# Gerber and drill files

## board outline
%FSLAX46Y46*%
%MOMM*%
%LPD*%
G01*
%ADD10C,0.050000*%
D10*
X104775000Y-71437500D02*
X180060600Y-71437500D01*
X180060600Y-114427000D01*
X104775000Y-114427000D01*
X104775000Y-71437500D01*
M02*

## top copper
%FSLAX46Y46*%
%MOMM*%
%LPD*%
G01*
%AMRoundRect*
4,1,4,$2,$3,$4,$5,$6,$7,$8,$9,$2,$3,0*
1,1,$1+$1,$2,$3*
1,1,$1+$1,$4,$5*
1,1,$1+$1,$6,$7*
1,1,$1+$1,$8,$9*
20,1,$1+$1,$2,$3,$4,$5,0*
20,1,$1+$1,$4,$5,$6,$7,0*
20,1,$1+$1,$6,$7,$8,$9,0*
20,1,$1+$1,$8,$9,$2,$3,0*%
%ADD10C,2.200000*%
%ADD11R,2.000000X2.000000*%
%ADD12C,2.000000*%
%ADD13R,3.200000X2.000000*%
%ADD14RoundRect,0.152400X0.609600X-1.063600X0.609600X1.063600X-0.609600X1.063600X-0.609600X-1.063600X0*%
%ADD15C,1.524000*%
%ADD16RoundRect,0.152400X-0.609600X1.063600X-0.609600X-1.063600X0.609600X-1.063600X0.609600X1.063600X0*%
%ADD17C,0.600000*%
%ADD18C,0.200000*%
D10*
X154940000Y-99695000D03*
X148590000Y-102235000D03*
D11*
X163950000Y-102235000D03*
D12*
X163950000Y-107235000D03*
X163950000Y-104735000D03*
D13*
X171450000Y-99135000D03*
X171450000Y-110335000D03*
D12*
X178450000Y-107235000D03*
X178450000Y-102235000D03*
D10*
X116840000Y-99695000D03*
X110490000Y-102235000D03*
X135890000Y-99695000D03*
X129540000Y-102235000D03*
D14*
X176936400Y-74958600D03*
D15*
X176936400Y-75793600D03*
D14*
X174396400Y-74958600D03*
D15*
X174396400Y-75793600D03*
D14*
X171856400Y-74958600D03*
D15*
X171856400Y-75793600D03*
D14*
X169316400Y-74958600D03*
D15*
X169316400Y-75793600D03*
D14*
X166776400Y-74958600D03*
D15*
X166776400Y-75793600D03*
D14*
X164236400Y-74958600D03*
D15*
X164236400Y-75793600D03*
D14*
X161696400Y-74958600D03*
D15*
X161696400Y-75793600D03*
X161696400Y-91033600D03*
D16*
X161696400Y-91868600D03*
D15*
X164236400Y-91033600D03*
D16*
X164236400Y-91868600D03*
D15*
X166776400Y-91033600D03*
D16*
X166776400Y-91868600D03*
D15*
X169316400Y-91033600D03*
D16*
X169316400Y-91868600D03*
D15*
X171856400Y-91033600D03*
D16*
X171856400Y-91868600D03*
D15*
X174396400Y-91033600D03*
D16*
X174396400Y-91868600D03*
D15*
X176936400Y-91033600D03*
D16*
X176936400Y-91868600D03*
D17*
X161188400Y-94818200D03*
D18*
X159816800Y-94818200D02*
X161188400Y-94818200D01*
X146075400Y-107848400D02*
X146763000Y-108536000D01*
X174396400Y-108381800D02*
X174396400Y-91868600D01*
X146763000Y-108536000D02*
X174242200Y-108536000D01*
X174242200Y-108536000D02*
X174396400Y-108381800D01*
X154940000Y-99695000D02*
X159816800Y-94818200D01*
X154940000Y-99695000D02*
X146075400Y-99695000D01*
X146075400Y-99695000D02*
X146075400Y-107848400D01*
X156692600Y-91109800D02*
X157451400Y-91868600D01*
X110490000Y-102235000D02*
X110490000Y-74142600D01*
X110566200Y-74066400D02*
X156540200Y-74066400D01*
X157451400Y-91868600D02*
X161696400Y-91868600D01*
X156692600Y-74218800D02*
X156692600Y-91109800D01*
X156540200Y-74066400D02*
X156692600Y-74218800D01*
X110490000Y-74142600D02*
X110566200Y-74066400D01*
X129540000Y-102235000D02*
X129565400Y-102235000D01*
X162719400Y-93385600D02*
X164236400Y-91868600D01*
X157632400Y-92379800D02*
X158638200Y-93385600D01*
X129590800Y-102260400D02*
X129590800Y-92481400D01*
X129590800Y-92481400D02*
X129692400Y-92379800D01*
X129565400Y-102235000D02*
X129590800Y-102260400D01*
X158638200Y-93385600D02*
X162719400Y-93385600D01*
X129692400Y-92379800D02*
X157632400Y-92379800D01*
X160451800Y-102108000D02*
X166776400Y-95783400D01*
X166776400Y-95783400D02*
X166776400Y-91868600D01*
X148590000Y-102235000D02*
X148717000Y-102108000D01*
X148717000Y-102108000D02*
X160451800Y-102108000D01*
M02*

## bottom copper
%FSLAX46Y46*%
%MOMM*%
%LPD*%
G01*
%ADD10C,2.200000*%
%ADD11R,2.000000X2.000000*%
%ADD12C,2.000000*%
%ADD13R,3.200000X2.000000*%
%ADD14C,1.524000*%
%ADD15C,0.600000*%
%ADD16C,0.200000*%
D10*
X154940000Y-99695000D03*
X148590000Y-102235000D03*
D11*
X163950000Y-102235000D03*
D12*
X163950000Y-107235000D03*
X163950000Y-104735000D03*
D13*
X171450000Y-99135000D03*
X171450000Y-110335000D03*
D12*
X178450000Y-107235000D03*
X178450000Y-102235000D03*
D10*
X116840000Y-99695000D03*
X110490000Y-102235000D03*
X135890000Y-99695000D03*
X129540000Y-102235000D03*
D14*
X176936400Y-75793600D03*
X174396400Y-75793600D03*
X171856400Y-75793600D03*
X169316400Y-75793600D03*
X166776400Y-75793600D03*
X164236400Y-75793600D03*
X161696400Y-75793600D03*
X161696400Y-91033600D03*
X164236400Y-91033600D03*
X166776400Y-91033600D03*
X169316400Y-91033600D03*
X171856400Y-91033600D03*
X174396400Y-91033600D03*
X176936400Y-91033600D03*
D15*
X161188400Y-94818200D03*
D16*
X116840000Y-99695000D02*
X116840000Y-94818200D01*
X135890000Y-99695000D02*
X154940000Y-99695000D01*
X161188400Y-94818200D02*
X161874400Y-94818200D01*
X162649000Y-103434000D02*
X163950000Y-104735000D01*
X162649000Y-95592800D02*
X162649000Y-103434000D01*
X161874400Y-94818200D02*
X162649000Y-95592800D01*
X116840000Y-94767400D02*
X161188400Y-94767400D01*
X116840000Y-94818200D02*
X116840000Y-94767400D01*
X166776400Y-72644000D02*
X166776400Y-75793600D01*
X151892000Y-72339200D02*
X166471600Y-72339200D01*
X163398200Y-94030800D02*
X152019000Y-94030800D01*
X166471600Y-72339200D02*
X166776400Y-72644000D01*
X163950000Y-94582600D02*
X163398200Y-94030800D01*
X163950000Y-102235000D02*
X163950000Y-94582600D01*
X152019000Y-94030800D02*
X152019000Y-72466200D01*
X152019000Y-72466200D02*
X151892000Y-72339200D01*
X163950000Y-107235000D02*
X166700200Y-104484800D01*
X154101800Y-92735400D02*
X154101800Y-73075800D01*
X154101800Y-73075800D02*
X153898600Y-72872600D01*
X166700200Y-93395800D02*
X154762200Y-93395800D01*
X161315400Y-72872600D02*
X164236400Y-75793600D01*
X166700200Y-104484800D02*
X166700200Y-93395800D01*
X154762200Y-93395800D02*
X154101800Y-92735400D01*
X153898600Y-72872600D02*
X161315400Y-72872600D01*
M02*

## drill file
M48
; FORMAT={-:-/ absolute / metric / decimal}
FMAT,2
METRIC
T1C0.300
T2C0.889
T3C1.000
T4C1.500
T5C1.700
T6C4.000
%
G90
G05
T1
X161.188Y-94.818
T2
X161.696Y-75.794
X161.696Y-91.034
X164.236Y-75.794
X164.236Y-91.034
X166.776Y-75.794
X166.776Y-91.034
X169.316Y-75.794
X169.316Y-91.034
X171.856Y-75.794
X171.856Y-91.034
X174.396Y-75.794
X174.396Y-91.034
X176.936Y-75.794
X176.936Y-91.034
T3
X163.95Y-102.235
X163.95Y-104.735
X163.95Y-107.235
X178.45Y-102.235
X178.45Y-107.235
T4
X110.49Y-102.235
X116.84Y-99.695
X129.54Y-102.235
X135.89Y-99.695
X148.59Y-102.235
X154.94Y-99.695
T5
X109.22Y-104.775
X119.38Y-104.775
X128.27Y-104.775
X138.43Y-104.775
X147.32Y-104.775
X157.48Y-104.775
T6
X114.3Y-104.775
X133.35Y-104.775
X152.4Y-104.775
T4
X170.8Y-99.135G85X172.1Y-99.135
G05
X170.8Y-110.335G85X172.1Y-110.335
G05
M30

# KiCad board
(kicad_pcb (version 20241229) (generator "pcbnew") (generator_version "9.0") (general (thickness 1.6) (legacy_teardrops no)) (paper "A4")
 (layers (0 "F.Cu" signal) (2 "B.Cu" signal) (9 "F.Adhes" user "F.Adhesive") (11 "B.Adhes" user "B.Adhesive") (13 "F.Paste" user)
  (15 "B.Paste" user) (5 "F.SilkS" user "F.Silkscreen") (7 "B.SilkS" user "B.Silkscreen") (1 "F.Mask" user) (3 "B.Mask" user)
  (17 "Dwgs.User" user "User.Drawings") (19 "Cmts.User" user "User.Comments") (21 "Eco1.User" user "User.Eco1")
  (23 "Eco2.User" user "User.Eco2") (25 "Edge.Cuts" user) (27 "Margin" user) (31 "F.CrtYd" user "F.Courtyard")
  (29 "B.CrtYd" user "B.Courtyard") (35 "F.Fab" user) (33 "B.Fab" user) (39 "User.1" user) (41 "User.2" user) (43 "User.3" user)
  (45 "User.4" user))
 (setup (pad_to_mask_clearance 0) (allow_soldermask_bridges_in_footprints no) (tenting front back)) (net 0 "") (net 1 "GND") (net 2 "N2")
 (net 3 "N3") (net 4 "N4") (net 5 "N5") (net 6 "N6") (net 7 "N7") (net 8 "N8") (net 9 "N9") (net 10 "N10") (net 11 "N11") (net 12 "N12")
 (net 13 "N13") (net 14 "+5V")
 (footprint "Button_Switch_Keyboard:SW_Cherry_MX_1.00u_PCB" (layer "F.Cu") (at 154.94 99.695)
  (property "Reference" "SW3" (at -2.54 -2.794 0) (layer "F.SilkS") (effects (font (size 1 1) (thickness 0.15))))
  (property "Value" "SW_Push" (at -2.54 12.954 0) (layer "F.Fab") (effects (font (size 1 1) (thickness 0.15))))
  (pad "" np_thru_hole circle (at -7.62 5.08) (size 1.7 1.7) (drill 1.7) (layers "*.Cu" "*.Mask"))
  (pad "" np_thru_hole circle (at -2.54 5.08) (size 4 4) (drill 4) (layers "*.Cu" "*.Mask"))
  (pad "" np_thru_hole circle (at 2.54 5.08) (size 1.7 1.7) (drill 1.7) (layers "*.Cu" "*.Mask"))
  (pad "1" thru_hole circle (at 0 0) (size 2.2 2.2) (drill 1.5) (layers "*.Cu" "*.Mask") (remove_unused_layers no) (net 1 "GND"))
  (pad "2" thru_hole circle (at -6.35 2.54) (size 2.2 2.2) (drill 1.5) (layers "*.Cu" "*.Mask") (remove_unused_layers no) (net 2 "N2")))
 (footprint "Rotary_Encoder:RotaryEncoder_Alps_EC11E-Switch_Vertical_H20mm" (layer "F.Cu") (at 163.95 102.235)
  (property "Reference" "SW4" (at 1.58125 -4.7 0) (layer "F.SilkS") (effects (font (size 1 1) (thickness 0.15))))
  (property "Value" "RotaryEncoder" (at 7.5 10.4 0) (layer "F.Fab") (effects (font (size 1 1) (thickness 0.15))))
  (pad "A" thru_hole rect (at 0 0) (size 2 2) (drill 1) (layers "*.Cu" "*.Mask") (remove_unused_layers no) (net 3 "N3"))
  (pad "B" thru_hole circle (at 0 5) (size 2 2) (drill 1) (layers "*.Cu" "*.Mask") (remove_unused_layers no) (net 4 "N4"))
  (pad "C" thru_hole circle (at 0 2.5) (size 2 2) (drill 1) (layers "*.Cu" "*.Mask") (remove_unused_layers no) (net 1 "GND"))
  (pad "MP" thru_hole rect (at 7.5 -3.1) (size 3.2 2) (drill oval 2.8 1.5) (layers "*.Cu" "*.Mask") (remove_unused_layers no))
  (pad "MP" thru_hole rect (at 7.5 8.1) (size 3.2 2) (drill oval 2.8 1.5) (layers "*.Cu" "*.Mask") (remove_unused_layers no))
  (pad "S1" thru_hole circle (at 14.5 5) (size 2 2) (drill 1) (layers "*.Cu" "*.Mask") (remove_unused_layers no))
  (pad "S2" thru_hole circle (at 14.5 0) (size 2 2) (drill 1) (layers "*.Cu" "*.Mask") (remove_unused_layers no)))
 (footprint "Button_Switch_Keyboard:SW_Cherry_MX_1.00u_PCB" (layer "F.Cu") (at 116.84 99.695)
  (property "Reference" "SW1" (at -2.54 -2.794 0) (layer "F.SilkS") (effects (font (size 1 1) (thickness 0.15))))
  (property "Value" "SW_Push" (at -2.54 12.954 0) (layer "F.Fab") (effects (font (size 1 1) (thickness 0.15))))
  (pad "" np_thru_hole circle (at -7.62 5.08) (size 1.7 1.7) (drill 1.7) (layers "*.Cu" "*.Mask"))
  (pad "" np_thru_hole circle (at -2.54 5.08) (size 4 4) (drill 4) (layers "*.Cu" "*.Mask"))
  (pad "" np_thru_hole circle (at 2.54 5.08) (size 1.7 1.7) (drill 1.7) (layers "*.Cu" "*.Mask"))
  (pad "1" thru_hole circle (at 0 0) (size 2.2 2.2) (drill 1.5) (layers "*.Cu" "*.Mask") (remove_unused_layers no) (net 1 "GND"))
  (pad "2" thru_hole circle (at -6.35 2.54) (size 2.2 2.2) (drill 1.5) (layers "*.Cu" "*.Mask") (remove_unused_layers no) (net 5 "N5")))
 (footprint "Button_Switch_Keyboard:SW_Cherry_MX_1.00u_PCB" (layer "F.Cu") (at 135.89 99.695)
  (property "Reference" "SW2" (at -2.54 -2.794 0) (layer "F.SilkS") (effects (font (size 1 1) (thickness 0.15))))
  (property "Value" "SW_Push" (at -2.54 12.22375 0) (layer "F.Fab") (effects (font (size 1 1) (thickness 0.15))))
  (pad "" np_thru_hole circle (at -7.62 5.08) (size 1.7 1.7) (drill 1.7) (layers "*.Cu" "*.Mask"))
  (pad "" np_thru_hole circle (at -2.54 5.08) (size 4 4) (drill 4) (layers "*.Cu" "*.Mask"))
  (pad "" np_thru_hole circle (at 2.54 5.08) (size 1.7 1.7) (drill 1.7) (layers "*.Cu" "*.Mask"))
  (pad "1" thru_hole circle (at 0 0) (size 2.2 2.2) (drill 1.5) (layers "*.Cu" "*.Mask") (remove_unused_layers no) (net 1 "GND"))
  (pad "2" thru_hole circle (at -6.35 2.54) (size 2.2 2.2) (drill 1.5) (layers "*.Cu" "*.Mask") (remove_unused_layers no) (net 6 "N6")))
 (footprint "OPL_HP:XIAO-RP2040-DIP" (layer "F.Cu") (at 169.3164 83.4136 -90)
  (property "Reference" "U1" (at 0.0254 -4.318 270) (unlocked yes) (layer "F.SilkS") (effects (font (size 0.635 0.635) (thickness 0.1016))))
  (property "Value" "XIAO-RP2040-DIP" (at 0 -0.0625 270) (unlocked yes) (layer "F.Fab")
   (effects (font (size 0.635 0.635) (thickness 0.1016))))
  (pad "1" smd roundrect (at -8.455 -7.62 90) (size 2.432 1.524) (layers "F.Cu" "F.Mask") (roundrect_rratio 0.1) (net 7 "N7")
   (thermal_bridge_angle 45))
  (pad "1" thru_hole circle (at -7.62 -7.62 90) (size 1.524 1.524) (drill 0.889) (layers "*.Cu" "*.Mask") (remove_unused_layers no)
   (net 7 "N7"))
  (pad "2" smd roundrect (at -8.455 -5.08 90) (size 2.432 1.524) (layers "F.Cu" "F.Mask") (roundrect_rratio 0.1) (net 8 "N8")
   (thermal_bridge_angle 45))
  (pad "2" thru_hole circle (at -7.62 -5.08 90) (size 1.524 1.524) (drill 0.889) (layers "*.Cu" "*.Mask") (remove_unused_layers no)
   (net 8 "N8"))
  (pad "3" smd roundrect (at -8.455 -2.54 90) (size 2.432 1.524) (layers "F.Cu" "F.Mask") (roundrect_rratio 0.1) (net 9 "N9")
   (thermal_bridge_angle 45))
  (pad "3" thru_hole circle (at -7.62 -2.54 90) (size 1.524 1.524) (drill 0.889) (layers "*.Cu" "*.Mask") (remove_unused_layers no)
   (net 9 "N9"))
  (pad "4" smd roundrect (at -8.455 0 90) (size 2.432 1.524) (layers "F.Cu" "F.Mask") (roundrect_rratio 0.1) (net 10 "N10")
   (thermal_bridge_angle 45))
  (pad "4" thru_hole circle (at -7.62 0 90) (size 1.524 1.524) (drill 0.889) (layers "*.Cu" "*.Mask") (remove_unused_layers no)
   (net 10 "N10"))
  (pad "5" smd roundrect (at -8.455 2.54 90) (size 2.432 1.524) (layers "F.Cu" "F.Mask") (roundrect_rratio 0.1) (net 3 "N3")
   (thermal_bridge_angle 45))
  (pad "5" thru_hole circle (at -7.62 2.54 90) (size 1.524 1.524) (drill 0.889) (layers "*.Cu" "*.Mask") (remove_unused_layers no)
   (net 3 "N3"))
  (pad "6" smd roundrect (at -8.455 5.08 90) (size 2.432 1.524) (layers "F.Cu" "F.Mask") (roundrect_rratio 0.1) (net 4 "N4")
   (thermal_bridge_angle 45))
  (pad "6" thru_hole circle (at -7.62 5.08 90) (size 1.524 1.524) (drill 0.889) (layers "*.Cu" "*.Mask") (remove_unused_layers no)
   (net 4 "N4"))
  (pad "7" smd roundrect (at -8.455 7.62 90) (size 2.432 1.524) (layers "F.Cu" "F.Mask") (roundrect_rratio 0.1) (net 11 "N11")
   (thermal_bridge_angle 45))
  (pad "7" thru_hole circle (at -7.62 7.62 90) (size 1.524 1.524) (drill 0.889) (layers "*.Cu" "*.Mask") (remove_unused_layers no)
   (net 11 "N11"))
  (pad "8" thru_hole circle (at 7.62 7.62 270) (size 1.524 1.524) (drill 0.889) (layers "*.Cu" "*.Mask") (remove_unused_layers no)
   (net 5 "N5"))
  (pad "8" smd roundrect (at 8.455 7.62 270) (size 2.432 1.524) (layers "F.Cu" "F.Mask") (roundrect_rratio 0.1) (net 5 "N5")
   (thermal_bridge_angle 45))
  (pad "9" thru_hole circle (at 7.62 5.08 270) (size 1.524 1.524) (drill 0.889) (layers "*.Cu" "*.Mask") (remove_unused_layers no)
   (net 6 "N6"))
  (pad "9" smd roundrect (at 8.455 5.08 270) (size 2.432 1.524) (layers "F.Cu" "F.Mask") (roundrect_rratio 0.1) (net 6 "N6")
   (thermal_bridge_angle 45))
  (pad "10" thru_hole circle (at 7.62 2.54 270) (size 1.524 1.524) (drill 0.889) (layers "*.Cu" "*.Mask") (remove_unused_layers no)
   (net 2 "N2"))
  (pad "10" smd roundrect (at 8.455 2.54 270) (size 2.432 1.524) (layers "F.Cu" "F.Mask") (roundrect_rratio 0.1) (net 2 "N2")
   (thermal_bridge_angle 45))
  (pad "11" thru_hole circle (at 7.62 0 270) (size 1.524 1.524) (drill 0.889) (layers "*.Cu" "*.Mask") (remove_unused_layers no)
   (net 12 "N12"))
  (pad "11" smd roundrect (at 8.455 0 270) (size 2.432 1.524) (layers "F.Cu" "F.Mask") (roundrect_rratio 0.1) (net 12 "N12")
   (thermal_bridge_angle 45))
  (pad "12" thru_hole circle (at 7.62 -2.54 270) (size 1.524 1.524) (drill 0.889) (layers "*.Cu" "*.Mask") (remove_unused_layers no)
   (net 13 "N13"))
  (pad "12" smd roundrect (at 8.455 -2.54 270) (size 2.432 1.524) (layers "F.Cu" "F.Mask") (roundrect_rratio 0.1) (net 13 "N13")
   (thermal_bridge_angle 45))
  (pad "13" thru_hole circle (at 7.62 -5.08 270) (size 1.524 1.524) (drill 0.889) (layers "*.Cu" "*.Mask") (remove_unused_layers no)
   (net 1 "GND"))
  (pad "13" smd roundrect (at 8.455 -5.08 270) (size 2.432 1.524) (layers "F.Cu" "F.Mask") (roundrect_rratio 0.1) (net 1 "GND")
   (thermal_bridge_angle 45))
  (pad "14" thru_hole circle (at 7.62 -7.62 270) (size 1.524 1.524) (drill 0.889) (layers "*.Cu" "*.Mask") (remove_unused_layers no)
   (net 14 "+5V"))
  (pad "14" smd roundrect (at 8.455 -7.62 270) (size 2.432 1.524) (layers "F.Cu" "F.Mask") (roundrect_rratio 0.1) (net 14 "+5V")
   (thermal_bridge_angle 45)))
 (gr_rect (start 104.775 71.4375) (end 180.0606 114.427) (stroke (width 0.05) (type default)) (fill no) (layer "Edge.Cuts"))
 (segment (start 159.8168 94.8182) (end 161.1884 94.8182) (width 0.2) (layer "F.Cu") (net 1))
 (segment (start 146.0754 107.8484) (end 146.763 108.536) (width 0.2) (layer "F.Cu") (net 1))
 (segment (start 174.3964 108.3818) (end 174.3964 91.8686) (width 0.2) (layer "F.Cu") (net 1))
 (segment (start 146.763 108.536) (end 174.2422 108.536) (width 0.2) (layer "F.Cu") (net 1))
 (segment (start 174.2422 108.536) (end 174.3964 108.3818) (width 0.2) (layer "F.Cu") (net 1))
 (segment (start 154.94 99.695) (end 159.8168 94.8182) (width 0.2) (layer "F.Cu") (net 1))
 (segment (start 154.94 99.695) (end 146.0754 99.695) (width 0.2) (layer "F.Cu") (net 1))
 (segment (start 146.0754 99.695) (end 146.0754 107.8484) (width 0.2) (layer "F.Cu") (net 1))
 (via (at 161.1884 94.8182) (size 0.6) (drill 0.3) (layers "F.Cu" "B.Cu") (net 1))
 (segment (start 116.84 99.695) (end 116.84 94.8182) (width 0.2) (layer "B.Cu") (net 1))
 (segment (start 135.89 99.695) (end 154.94 99.695) (width 0.2) (layer "B.Cu") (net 1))
 (segment (start 161.1884 94.8182) (end 161.8744 94.8182) (width 0.2) (layer "B.Cu") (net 1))
 (segment (start 162.649 103.434) (end 163.95 104.735) (width 0.2) (layer "B.Cu") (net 1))
 (segment (start 162.649 95.5928) (end 162.649 103.434) (width 0.2) (layer "B.Cu") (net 1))
 (segment (start 161.8744 94.8182) (end 162.649 95.5928) (width 0.2) (layer "B.Cu") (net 1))
 (segment (start 116.84 94.7674) (end 161.1884 94.7674) (width 0.2) (layer "B.Cu") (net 1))
 (segment (start 116.84 94.8182) (end 116.84 94.7674) (width 0.2) (layer "B.Cu") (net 1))
 (segment (start 166.7764 72.644) (end 166.7764 75.7936) (width 0.2) (layer "B.Cu") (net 3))
 (segment (start 151.892 72.3392) (end 166.4716 72.3392) (width 0.2) (layer "B.Cu") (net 3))
 (segment (start 163.3982 94.0308) (end 152.019 94.0308) (width 0.2) (layer "B.Cu") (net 3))
 (segment (start 166.4716 72.3392) (end 166.7764 72.644) (width 0.2) (layer "B.Cu") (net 3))
 (segment (start 163.95 94.5826) (end 163.3982 94.0308) (width 0.2) (layer "B.Cu") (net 3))
 (segment (start 163.95 102.235) (end 163.95 94.5826) (width 0.2) (layer "B.Cu") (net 3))
 (segment (start 152.019 94.0308) (end 152.019 72.4662) (width 0.2) (layer "B.Cu") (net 3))
 (segment (start 152.019 72.4662) (end 151.892 72.3392) (width 0.2) (layer "B.Cu") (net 3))
 (segment (start 163.95 107.235) (end 166.7002 104.4848) (width 0.2) (layer "B.Cu") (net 4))
 (segment (start 154.1018 92.7354) (end 154.1018 73.0758) (width 0.2) (layer "B.Cu") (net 4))
 (segment (start 154.1018 73.0758) (end 153.8986 72.8726) (width 0.2) (layer "B.Cu") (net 4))
 (segment (start 166.7002 93.3958) (end 154.7622 93.3958) (width 0.2) (layer "B.Cu") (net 4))
 (segment (start 161.3154 72.8726) (end 164.2364 75.7936) (width 0.2) (layer "B.Cu") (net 4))
 (segment (start 166.7002 104.4848) (end 166.7002 93.3958) (width 0.2) (layer "B.Cu") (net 4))
 (segment (start 154.7622 93.3958) (end 154.1018 92.7354) (width 0.2) (layer "B.Cu") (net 4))
 (segment (start 153.8986 72.8726) (end 161.3154 72.8726) (width 0.2) (layer "B.Cu") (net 4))
 (segment (start 156.6926 91.1098) (end 157.4514 91.8686) (width 0.2) (layer "F.Cu") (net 5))
 (segment (start 110.49 102.235) (end 110.49 74.1426) (width 0.2) (layer "F.Cu") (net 5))
 (segment (start 110.5662 74.0664) (end 156.5402 74.0664) (width 0.2) (layer "F.Cu") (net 5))
 (segment (start 157.4514 91.8686) (end 161.6964 91.8686) (width 0.2) (layer "F.Cu") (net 5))
 (segment (start 156.6926 74.2188) (end 156.6926 91.1098) (width 0.2) (layer "F.Cu") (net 5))
 (segment (start 156.5402 74.0664) (end 156.6926 74.2188) (width 0.2) (layer "F.Cu") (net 5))
 (segment (start 110.49 74.1426) (end 110.5662 74.0664) (width 0.2) (layer "F.Cu") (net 5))
 (segment (start 129.54 102.235) (end 129.5654 102.235) (width 0.2) (layer "F.Cu") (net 6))
 (segment (start 162.7194 93.3856) (end 164.2364 91.8686) (width 0.2) (layer "F.Cu") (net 6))
 (segment (start 157.6324 92.3798) (end 158.6382 93.3856) (width 0.2) (layer "F.Cu") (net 6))
 (segment (start 129.5908 102.2604) (end 129.5908 92.4814) (width 0.2) (layer "F.Cu") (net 6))
 (segment (start 129.5908 92.4814) (end 129.6924 92.3798) (width 0.2) (layer "F.Cu") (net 6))
 (segment (start 129.5654 102.235) (end 129.5908 102.2604) (width 0.2) (layer "F.Cu") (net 6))
 (segment (start 158.6382 93.3856) (end 162.7194 93.3856) (width 0.2) (layer "F.Cu") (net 6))
 (segment (start 129.6924 92.3798) (end 157.6324 92.3798) (width 0.2) (layer "F.Cu") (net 6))
 (segment (start 160.4518 102.108) (end 166.7764 95.7834) (width 0.2) (layer "F.Cu") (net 2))
 (segment (start 166.7764 95.7834) (end 166.7764 91.8686) (width 0.2) (layer "F.Cu") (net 2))
 (segment (start 148.59 102.235) (end 148.717 102.108) (width 0.2) (layer "F.Cu") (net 2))
 (segment (start 148.717 102.108) (end 160.4518 102.108) (width 0.2) (layer "F.Cu") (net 2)))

